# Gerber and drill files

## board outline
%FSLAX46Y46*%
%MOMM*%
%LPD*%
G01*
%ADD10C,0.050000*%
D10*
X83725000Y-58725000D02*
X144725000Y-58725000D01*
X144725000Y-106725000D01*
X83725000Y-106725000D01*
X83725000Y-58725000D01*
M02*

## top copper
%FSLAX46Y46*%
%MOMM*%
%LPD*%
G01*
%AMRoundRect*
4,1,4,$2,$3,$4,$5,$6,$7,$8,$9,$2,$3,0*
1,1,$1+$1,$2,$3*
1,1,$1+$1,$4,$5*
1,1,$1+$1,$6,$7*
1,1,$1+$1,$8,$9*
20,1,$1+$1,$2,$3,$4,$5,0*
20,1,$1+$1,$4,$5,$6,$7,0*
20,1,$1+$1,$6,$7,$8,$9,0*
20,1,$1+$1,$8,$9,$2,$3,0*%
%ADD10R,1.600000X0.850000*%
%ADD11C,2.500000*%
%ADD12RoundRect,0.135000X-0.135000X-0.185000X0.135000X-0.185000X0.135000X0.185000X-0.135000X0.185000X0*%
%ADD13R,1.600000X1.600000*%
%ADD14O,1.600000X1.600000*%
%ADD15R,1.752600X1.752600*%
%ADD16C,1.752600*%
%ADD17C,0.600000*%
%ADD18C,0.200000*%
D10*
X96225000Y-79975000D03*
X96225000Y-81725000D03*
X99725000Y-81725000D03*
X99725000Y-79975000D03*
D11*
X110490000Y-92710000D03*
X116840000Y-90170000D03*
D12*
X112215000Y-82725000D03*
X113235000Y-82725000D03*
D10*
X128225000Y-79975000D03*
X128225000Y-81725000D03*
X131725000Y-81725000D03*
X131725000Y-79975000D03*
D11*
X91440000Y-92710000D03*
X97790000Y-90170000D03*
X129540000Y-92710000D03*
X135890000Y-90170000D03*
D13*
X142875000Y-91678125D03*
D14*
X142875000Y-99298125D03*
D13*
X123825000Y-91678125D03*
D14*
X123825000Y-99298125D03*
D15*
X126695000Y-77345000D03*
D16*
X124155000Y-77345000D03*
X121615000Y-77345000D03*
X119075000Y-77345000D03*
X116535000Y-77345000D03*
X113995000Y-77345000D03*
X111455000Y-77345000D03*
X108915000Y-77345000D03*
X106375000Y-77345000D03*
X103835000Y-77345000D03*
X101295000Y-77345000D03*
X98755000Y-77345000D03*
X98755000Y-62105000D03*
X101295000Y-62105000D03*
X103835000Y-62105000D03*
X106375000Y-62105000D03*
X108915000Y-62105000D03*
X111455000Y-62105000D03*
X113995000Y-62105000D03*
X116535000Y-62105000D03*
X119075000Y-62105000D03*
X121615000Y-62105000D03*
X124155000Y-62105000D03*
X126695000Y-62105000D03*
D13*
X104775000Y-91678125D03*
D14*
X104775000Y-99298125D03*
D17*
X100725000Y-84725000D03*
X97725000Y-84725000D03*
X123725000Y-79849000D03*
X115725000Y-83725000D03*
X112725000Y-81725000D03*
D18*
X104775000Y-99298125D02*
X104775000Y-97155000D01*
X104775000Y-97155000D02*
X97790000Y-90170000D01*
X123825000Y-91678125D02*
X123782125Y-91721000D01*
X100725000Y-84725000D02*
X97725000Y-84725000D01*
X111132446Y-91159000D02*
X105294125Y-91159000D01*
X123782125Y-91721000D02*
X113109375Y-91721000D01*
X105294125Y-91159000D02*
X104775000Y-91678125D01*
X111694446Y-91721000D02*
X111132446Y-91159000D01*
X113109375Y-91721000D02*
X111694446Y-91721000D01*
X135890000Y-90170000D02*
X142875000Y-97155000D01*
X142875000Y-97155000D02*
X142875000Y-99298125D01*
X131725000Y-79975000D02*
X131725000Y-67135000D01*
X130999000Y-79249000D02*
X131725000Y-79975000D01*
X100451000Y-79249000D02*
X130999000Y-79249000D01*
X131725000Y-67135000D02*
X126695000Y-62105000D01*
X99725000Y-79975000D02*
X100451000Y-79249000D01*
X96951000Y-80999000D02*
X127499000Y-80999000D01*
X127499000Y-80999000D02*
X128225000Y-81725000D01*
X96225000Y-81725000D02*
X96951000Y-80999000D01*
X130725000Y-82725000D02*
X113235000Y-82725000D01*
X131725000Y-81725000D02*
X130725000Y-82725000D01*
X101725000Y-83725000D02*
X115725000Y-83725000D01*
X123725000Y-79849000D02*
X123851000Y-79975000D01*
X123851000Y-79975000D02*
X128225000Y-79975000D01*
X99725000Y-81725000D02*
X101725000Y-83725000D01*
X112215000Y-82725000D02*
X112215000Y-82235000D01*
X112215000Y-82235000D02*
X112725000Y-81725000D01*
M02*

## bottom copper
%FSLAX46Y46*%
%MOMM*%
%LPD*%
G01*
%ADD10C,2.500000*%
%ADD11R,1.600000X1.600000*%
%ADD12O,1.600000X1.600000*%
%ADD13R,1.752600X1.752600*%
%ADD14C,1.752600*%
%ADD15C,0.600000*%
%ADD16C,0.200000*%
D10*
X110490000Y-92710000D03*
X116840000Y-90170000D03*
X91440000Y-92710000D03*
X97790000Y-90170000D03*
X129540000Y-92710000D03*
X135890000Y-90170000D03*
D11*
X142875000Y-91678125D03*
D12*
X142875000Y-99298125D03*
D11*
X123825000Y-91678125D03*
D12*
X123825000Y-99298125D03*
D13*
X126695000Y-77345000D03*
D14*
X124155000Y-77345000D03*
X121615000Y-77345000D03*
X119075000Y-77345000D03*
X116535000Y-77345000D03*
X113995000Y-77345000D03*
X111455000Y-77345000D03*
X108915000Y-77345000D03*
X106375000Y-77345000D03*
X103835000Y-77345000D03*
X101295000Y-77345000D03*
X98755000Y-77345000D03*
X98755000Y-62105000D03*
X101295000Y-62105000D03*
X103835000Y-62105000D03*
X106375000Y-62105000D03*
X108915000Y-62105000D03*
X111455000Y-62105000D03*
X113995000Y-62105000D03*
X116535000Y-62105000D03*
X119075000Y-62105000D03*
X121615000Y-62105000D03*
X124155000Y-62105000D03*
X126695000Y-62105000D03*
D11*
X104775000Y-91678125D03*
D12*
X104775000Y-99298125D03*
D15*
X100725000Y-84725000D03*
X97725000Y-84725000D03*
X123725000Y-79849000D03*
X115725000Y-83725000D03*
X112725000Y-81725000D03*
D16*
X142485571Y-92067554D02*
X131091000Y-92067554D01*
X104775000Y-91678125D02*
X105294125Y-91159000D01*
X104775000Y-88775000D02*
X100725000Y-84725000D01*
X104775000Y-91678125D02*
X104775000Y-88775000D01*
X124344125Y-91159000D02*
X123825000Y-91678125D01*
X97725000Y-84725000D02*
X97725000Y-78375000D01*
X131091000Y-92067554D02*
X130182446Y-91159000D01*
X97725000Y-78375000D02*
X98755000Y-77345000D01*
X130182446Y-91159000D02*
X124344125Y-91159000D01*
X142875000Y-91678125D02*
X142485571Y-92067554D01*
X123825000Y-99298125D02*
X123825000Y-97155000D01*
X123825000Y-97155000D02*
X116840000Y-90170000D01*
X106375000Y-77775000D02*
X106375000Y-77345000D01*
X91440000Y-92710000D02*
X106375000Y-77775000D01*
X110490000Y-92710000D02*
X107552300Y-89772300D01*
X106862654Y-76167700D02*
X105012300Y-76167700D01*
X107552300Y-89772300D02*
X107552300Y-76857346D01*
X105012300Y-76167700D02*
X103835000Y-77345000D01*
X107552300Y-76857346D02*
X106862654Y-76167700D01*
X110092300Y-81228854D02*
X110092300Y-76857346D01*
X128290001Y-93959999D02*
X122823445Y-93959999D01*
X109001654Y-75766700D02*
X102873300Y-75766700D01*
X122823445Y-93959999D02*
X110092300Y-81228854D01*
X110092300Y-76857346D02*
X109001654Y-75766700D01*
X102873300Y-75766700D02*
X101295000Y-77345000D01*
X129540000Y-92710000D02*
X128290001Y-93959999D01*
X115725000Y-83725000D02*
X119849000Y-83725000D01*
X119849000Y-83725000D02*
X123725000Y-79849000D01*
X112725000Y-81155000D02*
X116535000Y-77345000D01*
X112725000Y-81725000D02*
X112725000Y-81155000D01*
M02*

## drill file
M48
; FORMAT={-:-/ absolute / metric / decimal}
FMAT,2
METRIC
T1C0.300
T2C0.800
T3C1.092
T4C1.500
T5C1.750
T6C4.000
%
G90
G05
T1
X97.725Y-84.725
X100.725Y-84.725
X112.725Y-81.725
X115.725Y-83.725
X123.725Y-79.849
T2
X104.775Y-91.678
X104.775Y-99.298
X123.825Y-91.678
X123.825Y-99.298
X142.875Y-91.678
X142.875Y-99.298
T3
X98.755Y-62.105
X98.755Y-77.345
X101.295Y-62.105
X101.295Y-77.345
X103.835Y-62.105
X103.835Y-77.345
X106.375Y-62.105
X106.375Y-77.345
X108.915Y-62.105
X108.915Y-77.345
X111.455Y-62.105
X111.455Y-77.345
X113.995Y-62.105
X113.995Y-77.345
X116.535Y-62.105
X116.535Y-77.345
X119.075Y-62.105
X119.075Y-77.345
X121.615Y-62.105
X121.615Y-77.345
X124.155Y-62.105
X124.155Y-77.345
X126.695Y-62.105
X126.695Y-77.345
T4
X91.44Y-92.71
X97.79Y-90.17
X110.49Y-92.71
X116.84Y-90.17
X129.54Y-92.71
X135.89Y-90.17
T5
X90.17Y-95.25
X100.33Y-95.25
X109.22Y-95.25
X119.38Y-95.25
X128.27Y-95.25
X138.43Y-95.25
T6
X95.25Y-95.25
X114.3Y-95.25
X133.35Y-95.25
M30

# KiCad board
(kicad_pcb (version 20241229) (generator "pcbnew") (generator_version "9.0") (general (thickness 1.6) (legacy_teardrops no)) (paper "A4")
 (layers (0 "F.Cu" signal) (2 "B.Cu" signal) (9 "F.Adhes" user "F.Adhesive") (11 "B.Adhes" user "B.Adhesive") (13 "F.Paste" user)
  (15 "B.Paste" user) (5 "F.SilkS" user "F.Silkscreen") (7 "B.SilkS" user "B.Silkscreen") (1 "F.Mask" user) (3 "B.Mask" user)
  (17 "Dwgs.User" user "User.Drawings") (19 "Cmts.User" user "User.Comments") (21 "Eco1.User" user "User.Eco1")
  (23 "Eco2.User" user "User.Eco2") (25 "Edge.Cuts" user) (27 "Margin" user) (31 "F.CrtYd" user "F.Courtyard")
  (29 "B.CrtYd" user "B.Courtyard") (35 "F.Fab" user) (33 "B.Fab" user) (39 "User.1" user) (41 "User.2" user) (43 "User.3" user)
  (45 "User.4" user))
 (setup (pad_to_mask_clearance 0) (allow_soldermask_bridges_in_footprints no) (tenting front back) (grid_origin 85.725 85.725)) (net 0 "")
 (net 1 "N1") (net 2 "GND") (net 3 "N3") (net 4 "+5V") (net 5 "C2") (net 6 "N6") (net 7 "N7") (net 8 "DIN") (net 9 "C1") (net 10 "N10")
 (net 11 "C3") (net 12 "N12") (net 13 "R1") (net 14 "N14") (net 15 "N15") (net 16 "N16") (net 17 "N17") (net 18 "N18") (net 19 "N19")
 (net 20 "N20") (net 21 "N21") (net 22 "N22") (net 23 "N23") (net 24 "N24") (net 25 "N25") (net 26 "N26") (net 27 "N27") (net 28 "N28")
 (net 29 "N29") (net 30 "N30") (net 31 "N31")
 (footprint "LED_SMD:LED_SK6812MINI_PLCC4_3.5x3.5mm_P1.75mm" (layer "F.Cu") (at 97.975 80.85)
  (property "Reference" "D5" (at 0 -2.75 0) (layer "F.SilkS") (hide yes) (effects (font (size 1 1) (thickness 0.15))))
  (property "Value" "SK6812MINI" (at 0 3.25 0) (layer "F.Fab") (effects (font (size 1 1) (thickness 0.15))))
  (pad "1" smd rect (at -1.75 -0.875) (size 1.6 0.85) (layers "F.Cu" "F.Mask" "F.Paste") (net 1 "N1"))
  (pad "2" smd rect (at -1.75 0.875) (size 1.6 0.85) (layers "F.Cu" "F.Mask" "F.Paste") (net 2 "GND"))
  (pad "3" smd rect (at 1.75 0.875) (size 1.6 0.85) (layers "F.Cu" "F.Mask" "F.Paste") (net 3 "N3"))
  (pad "4" smd rect (at 1.75 -0.875) (size 1.6 0.85) (layers "F.Cu" "F.Mask" "F.Paste") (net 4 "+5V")))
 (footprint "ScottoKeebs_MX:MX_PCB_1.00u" (layer "F.Cu") (at 114.3 95.25)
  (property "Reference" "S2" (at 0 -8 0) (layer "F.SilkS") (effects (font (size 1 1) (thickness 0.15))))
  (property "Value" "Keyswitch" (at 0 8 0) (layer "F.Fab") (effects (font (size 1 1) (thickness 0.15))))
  (pad "" np_thru_hole circle (at -5.08 0) (size 1.75 1.75) (drill 1.75) (layers "*.Cu" "*.Mask"))
  (pad "" np_thru_hole circle (at 0 0) (size 4 4) (drill 4) (layers "*.Cu" "*.Mask"))
  (pad "" np_thru_hole circle (at 5.08 0) (size 1.75 1.75) (drill 1.75) (layers "*.Cu" "*.Mask"))
  (pad "1" thru_hole circle (at -3.81 -2.54) (size 2.5 2.5) (drill 1.5) (layers "*.Cu" "*.Mask") (remove_unused_layers no) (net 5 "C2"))
  (pad "2" thru_hole circle (at 2.54 -5.08) (size 2.5 2.5) (drill 1.5) (layers "*.Cu" "*.Mask") (remove_unused_layers no) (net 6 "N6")))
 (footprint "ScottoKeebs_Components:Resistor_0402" (layer "F.Cu") (at 112.725 82.725)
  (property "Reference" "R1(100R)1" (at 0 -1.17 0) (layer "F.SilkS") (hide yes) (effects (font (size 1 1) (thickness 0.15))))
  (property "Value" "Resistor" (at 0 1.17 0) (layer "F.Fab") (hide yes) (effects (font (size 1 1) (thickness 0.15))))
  (pad "1" smd roundrect (at -0.51 0) (size 0.54 0.64) (layers "F.Cu" "F.Mask" "F.Paste") (roundrect_rratio 0.25) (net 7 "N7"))
  (pad "2" smd roundrect (at 0.51 0) (size 0.54 0.64) (layers "F.Cu" "F.Mask" "F.Paste") (roundrect_rratio 0.25) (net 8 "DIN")))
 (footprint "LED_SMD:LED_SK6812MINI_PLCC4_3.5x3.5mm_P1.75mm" (layer "F.Cu") (at 129.975 80.85)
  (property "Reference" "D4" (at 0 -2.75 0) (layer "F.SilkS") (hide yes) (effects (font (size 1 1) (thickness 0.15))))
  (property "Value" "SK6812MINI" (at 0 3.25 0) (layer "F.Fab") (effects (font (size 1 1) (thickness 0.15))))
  (pad "1" smd rect (at -1.75 -0.875) (size 1.6 0.85) (layers "F.Cu" "F.Mask" "F.Paste") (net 3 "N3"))
  (pad "2" smd rect (at -1.75 0.875) (size 1.6 0.85) (layers "F.Cu" "F.Mask" "F.Paste") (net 2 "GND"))
  (pad "3" smd rect (at 1.75 0.875) (size 1.6 0.85) (layers "F.Cu" "F.Mask" "F.Paste") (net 8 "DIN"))
  (pad "4" smd rect (at 1.75 -0.875) (size 1.6 0.85) (layers "F.Cu" "F.Mask" "F.Paste") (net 4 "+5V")))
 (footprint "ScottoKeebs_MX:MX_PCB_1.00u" (layer "F.Cu") (at 95.25 95.25)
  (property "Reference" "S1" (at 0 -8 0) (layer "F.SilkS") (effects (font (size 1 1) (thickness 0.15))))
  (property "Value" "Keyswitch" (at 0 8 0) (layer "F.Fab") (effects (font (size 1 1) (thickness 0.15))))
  (pad "" np_thru_hole circle (at -5.08 0) (size 1.75 1.75) (drill 1.75) (layers "*.Cu" "*.Mask"))
  (pad "" np_thru_hole circle (at 0 0) (size 4 4) (drill 4) (layers "*.Cu" "*.Mask"))
  (pad "" np_thru_hole circle (at 5.08 0) (size 1.75 1.75) (drill 1.75) (layers "*.Cu" "*.Mask"))
  (pad "1" thru_hole circle (at -3.81 -2.54) (size 2.5 2.5) (drill 1.5) (layers "*.Cu" "*.Mask") (remove_unused_layers no) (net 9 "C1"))
  (pad "2" thru_hole circle (at 2.54 -5.08) (size 2.5 2.5) (drill 1.5) (layers "*.Cu" "*.Mask") (remove_unused_layers no) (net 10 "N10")))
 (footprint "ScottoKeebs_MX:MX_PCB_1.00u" (layer "F.Cu") (at 133.35 95.25)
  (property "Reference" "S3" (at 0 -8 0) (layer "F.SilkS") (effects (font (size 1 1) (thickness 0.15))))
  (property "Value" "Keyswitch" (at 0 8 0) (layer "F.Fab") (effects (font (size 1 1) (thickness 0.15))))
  (pad "" np_thru_hole circle (at -5.08 0) (size 1.75 1.75) (drill 1.75) (layers "*.Cu" "*.Mask"))
  (pad "" np_thru_hole circle (at 0 0) (size 4 4) (drill 4) (layers "*.Cu" "*.Mask"))
  (pad "" np_thru_hole circle (at 5.08 0) (size 1.75 1.75) (drill 1.75) (layers "*.Cu" "*.Mask"))
  (pad "1" thru_hole circle (at -3.81 -2.54) (size 2.5 2.5) (drill 1.5) (layers "*.Cu" "*.Mask") (remove_unused_layers no) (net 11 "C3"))
  (pad "2" thru_hole circle (at 2.54 -5.08) (size 2.5 2.5) (drill 1.5) (layers "*.Cu" "*.Mask") (remove_unused_layers no) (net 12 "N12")))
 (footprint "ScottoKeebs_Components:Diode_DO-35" (layer "B.Cu") (at 142.875 91.678125 -90)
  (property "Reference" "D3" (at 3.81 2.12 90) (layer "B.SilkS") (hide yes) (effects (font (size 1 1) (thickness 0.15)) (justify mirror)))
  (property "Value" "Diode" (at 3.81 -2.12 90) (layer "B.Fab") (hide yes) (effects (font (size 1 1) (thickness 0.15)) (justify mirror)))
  (pad "1" thru_hole rect (at 0 0 270) (size 1.6 1.6) (drill 0.8) (layers "*.Cu" "*.Mask") (remove_unused_layers no) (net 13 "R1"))
  (pad "2" thru_hole oval (at 7.62 0 270) (size 1.6 1.6) (drill 0.8) (layers "*.Cu" "*.Mask") (remove_unused_layers no) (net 12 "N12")))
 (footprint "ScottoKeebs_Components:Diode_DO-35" (layer "B.Cu") (at 123.825 91.678125 -90)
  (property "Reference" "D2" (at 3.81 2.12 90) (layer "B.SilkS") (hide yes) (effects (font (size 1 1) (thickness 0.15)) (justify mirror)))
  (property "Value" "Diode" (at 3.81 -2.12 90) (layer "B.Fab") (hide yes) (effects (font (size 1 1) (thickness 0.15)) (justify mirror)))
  (pad "1" thru_hole rect (at 0 0 270) (size 1.6 1.6) (drill 0.8) (layers "*.Cu" "*.Mask") (remove_unused_layers no) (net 13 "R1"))
  (pad "2" thru_hole oval (at 7.62 0 270) (size 1.6 1.6) (drill 0.8) (layers "*.Cu" "*.Mask") (remove_unused_layers no) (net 6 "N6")))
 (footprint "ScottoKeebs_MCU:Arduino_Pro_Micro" (layer "B.Cu") (at 112.725 69.725 90)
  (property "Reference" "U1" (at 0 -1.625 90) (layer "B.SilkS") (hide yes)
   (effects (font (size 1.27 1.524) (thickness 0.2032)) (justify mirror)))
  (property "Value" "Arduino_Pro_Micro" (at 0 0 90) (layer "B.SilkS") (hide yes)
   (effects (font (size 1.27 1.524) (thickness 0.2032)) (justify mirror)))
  (pad "1" thru_hole rect (at -7.62 13.97 180) (size 1.7526 1.7526) (drill 1.0922) (layers "*.Cu" "*.SilkS" "*.Mask")
   (remove_unused_layers no) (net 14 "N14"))
  (pad "2" thru_hole circle (at -7.62 11.43 180) (size 1.7526 1.7526) (drill 1.0922) (layers "*.Cu" "*.SilkS" "*.Mask")
   (remove_unused_layers no) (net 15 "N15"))
  (pad "3" thru_hole circle (at -7.62 8.89 180) (size 1.7526 1.7526) (drill 1.0922) (layers "*.Cu" "*.SilkS" "*.Mask")
   (remove_unused_layers no) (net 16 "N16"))
  (pad "4" thru_hole circle (at -7.62 6.35 180) (size 1.7526 1.7526) (drill 1.0922) (layers "*.Cu" "*.SilkS" "*.Mask")
   (remove_unused_layers no) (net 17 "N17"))
  (pad "5" thru_hole circle (at -7.62 3.81 180) (size 1.7526 1.7526) (drill 1.0922) (layers "*.Cu" "*.SilkS" "*.Mask")
   (remove_unused_layers no) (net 7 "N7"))
  (pad "6" thru_hole circle (at -7.62 1.27 180) (size 1.7526 1.7526) (drill 1.0922) (layers "*.Cu" "*.SilkS" "*.Mask")
   (remove_unused_layers no) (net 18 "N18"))
  (pad "7" thru_hole circle (at -7.62 -1.27 180) (size 1.7526 1.7526) (drill 1.0922) (layers "*.Cu" "*.SilkS" "*.Mask")
   (remove_unused_layers no) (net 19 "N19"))
  (pad "8" thru_hole circle (at -7.62 -3.81 180) (size 1.7526 1.7526) (drill 1.0922) (layers "*.Cu" "*.SilkS" "*.Mask")
   (remove_unused_layers no) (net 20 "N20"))
  (pad "9" thru_hole circle (at -7.62 -6.35 180) (size 1.7526 1.7526) (drill 1.0922) (layers "*.Cu" "*.SilkS" "*.Mask")
   (remove_unused_layers no) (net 9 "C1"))
  (pad "10" thru_hole circle (at -7.62 -8.89 180) (size 1.7526 1.7526) (drill 1.0922) (layers "*.Cu" "*.SilkS" "*.Mask")
   (remove_unused_layers no) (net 5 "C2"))
  (pad "11" thru_hole circle (at -7.62 -11.43 180) (size 1.7526 1.7526) (drill 1.0922) (layers "*.Cu" "*.SilkS" "*.Mask")
   (remove_unused_layers no) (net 11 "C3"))
  (pad "12" thru_hole circle (at -7.62 -13.97 180) (size 1.7526 1.7526) (drill 1.0922) (layers "*.Cu" "*.SilkS" "*.Mask")
   (remove_unused_layers no) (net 13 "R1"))
  (pad "13" thru_hole circle (at 7.62 -13.97 180) (size 1.7526 1.7526) (drill 1.0922) (layers "*.Cu" "*.SilkS" "*.Mask")
   (remove_unused_layers no) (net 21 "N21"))
  (pad "14" thru_hole circle (at 7.62 -11.43 180) (size 1.7526 1.7526) (drill 1.0922) (layers "*.Cu" "*.SilkS" "*.Mask")
   (remove_unused_layers no) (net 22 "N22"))
  (pad "15" thru_hole circle (at 7.62 -8.89 180) (size 1.7526 1.7526) (drill 1.0922) (layers "*.Cu" "*.SilkS" "*.Mask")
   (remove_unused_layers no) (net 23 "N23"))
  (pad "16" thru_hole circle (at 7.62 -6.35 180) (size 1.7526 1.7526) (drill 1.0922) (layers "*.Cu" "*.SilkS" "*.Mask")
   (remove_unused_layers no) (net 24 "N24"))
  (pad "17" thru_hole circle (at 7.62 -3.81 180) (size 1.7526 1.7526) (drill 1.0922) (layers "*.Cu" "*.SilkS" "*.Mask")
   (remove_unused_layers no) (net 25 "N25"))
  (pad "18" thru_hole circle (at 7.62 -1.27 180) (size 1.7526 1.7526) (drill 1.0922) (layers "*.Cu" "*.SilkS" "*.Mask")
   (remove_unused_layers no) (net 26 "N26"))
  (pad "19" thru_hole circle (at 7.62 1.27 180) (size 1.7526 1.7526) (drill 1.0922) (layers "*.Cu" "*.SilkS" "*.Mask")
   (remove_unused_layers no) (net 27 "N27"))
  (pad "20" thru_hole circle (at 7.62 3.81 180) (size 1.7526 1.7526) (drill 1.0922) (layers "*.Cu" "*.SilkS" "*.Mask")
   (remove_unused_layers no) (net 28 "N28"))
  (pad "21" thru_hole circle (at 7.62 6.35 180) (size 1.7526 1.7526) (drill 1.0922) (layers "*.Cu" "*.SilkS" "*.Mask")
   (remove_unused_layers no) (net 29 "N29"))
  (pad "22" thru_hole circle (at 7.62 8.89 180) (size 1.7526 1.7526) (drill 1.0922) (layers "*.Cu" "*.SilkS" "*.Mask")
   (remove_unused_layers no) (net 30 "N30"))
  (pad "23" thru_hole circle (at 7.62 11.43 180) (size 1.7526 1.7526) (drill 1.0922) (layers "*.Cu" "*.SilkS" "*.Mask")
   (remove_unused_layers no) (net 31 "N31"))
  (pad "24" thru_hole circle (at 7.62 13.97 180) (size 1.7526 1.7526) (drill 1.0922) (layers "*.Cu" "*.SilkS" "*.Mask")
   (remove_unused_layers no) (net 4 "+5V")))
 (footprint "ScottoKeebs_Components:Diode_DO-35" (layer "B.Cu") (at 104.775 91.678125 -90)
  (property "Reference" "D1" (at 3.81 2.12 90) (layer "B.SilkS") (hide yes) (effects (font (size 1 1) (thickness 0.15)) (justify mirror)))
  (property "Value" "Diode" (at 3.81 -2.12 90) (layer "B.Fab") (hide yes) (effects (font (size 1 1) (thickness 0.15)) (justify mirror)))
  (pad "1" thru_hole rect (at 0 0 270) (size 1.6 1.6) (drill 0.8) (layers "*.Cu" "*.Mask") (remove_unused_layers no) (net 13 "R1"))
  (pad "2" thru_hole oval (at 7.62 0 270) (size 1.6 1.6) (drill 0.8) (layers "*.Cu" "*.Mask") (remove_unused_layers no) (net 10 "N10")))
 (gr_rect (start 83.725 58.725) (end 144.725 106.725) (stroke (width 0.05) (type default)) (fill no) (layer "Edge.Cuts"))
 (segment (start 104.775 99.298125) (end 104.775 97.155) (width 0.2) (layer "F.Cu") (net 10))
 (segment (start 104.775 97.155) (end 97.79 90.17) (width 0.2) (layer "F.Cu") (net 10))
 (segment (start 123.825 91.678125) (end 123.782125 91.721) (width 0.2) (layer "F.Cu") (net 13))
 (segment (start 100.725 84.725) (end 97.725 84.725) (width 0.2) (layer "F.Cu") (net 13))
 (segment (start 111.132446 91.159) (end 105.294125 91.159) (width 0.2) (layer "F.Cu") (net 13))
 (segment (start 123.782125 91.721) (end 113.109375 91.721) (width 0.2) (layer "F.Cu") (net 13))
 (segment (start 105.294125 91.159) (end 104.775 91.678125) (width 0.2) (layer "F.Cu") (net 13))
 (segment (start 111.694446 91.721) (end 111.132446 91.159) (width 0.2) (layer "F.Cu") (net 13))
 (segment (start 113.109375 91.721) (end 111.694446 91.721) (width 0.2) (layer "F.Cu") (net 13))
 (via (at 100.725 84.725) (size 0.6) (drill 0.3) (layers "F.Cu" "B.Cu") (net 13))
 (via (at 97.725 84.725) (size 0.6) (drill 0.3) (layers "F.Cu" "B.Cu") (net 13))
 (segment (start 142.485571 92.067554) (end 131.091 92.067554) (width 0.2) (layer "B.Cu") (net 13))
 (segment (start 104.775 91.678125) (end 105.294125 91.159) (width 0.2) (layer "B.Cu") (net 13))
 (segment (start 104.775 88.775) (end 100.725 84.725) (width 0.2) (layer "B.Cu") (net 13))
 (segment (start 104.775 91.678125) (end 104.775 88.775) (width 0.2) (layer "B.Cu") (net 13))
 (segment (start 124.344125 91.159) (end 123.825 91.678125) (width 0.2) (layer "B.Cu") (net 13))
 (segment (start 97.725 84.725) (end 97.725 78.375) (width 0.2) (layer "B.Cu") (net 13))
 (segment (start 131.091 92.067554) (end 130.182446 91.159) (width 0.2) (layer "B.Cu") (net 13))
 (segment (start 97.725 78.375) (end 98.755 77.345) (width 0.2) (layer "B.Cu") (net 13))
 (segment (start 130.182446 91.159) (end 124.344125 91.159) (width 0.2) (layer "B.Cu") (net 13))
 (segment (start 142.875 91.678125) (end 142.485571 92.067554) (width 0.2) (layer "B.Cu") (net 13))
 (segment (start 123.825 99.298125) (end 123.825 97.155) (width 0.2) (layer "B.Cu") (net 6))
 (segment (start 123.825 97.155) (end 116.84 90.17) (width 0.2) (layer "B.Cu") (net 6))
 (segment (start 135.89 90.17) (end 142.875 97.155) (width 0.2) (layer "F.Cu") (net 12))
 (segment (start 142.875 97.155) (end 142.875 99.298125) (width 0.2) (layer "F.Cu") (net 12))
 (segment (start 106.375 77.775) (end 106.375 77.345) (width 0.2) (layer "B.Cu") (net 9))
 (segment (start 91.44 92.71) (end 106.375 77.775) (width 0.2) (layer "B.Cu") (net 9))
 (segment (start 110.49 92.71) (end 107.5523 89.7723) (width 0.2) (layer "B.Cu") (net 5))
 (segment (start 106.862654 76.1677) (end 105.0123 76.1677) (width 0.2) (layer "B.Cu") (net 5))
 (segment (start 107.5523 89.7723) (end 107.5523 76.857346) (width 0.2) (layer "B.Cu") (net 5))
 (segment (start 105.0123 76.1677) (end 103.835 77.345) (width 0.2) (layer "B.Cu") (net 5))
 (segment (start 107.5523 76.857346) (end 106.862654 76.1677) (width 0.2) (layer "B.Cu") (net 5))
 (segment (start 110.0923 81.228854) (end 110.0923 76.857346) (width 0.2) (layer "B.Cu") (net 11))
 (segment (start 128.290001 93.959999) (end 122.823445 93.959999) (width 0.2) (layer "B.Cu") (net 11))
 (segment (start 109.001654 75.7667) (end 102.8733 75.7667) (width 0.2) (layer "B.Cu") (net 11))
 (segment (start 122.823445 93.959999) (end 110.0923 81.228854) (width 0.2) (layer "B.Cu") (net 11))
 (segment (start 110.0923 76.857346) (end 109.001654 75.7667) (width 0.2) (layer "B.Cu") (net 11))
 (segment (start 102.8733 75.7667) (end 101.295 77.345) (width 0.2) (layer "B.Cu") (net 11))
 (segment (start 129.54 92.71) (end 128.290001 93.959999) (width 0.2) (layer "B.Cu") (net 11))
 (segment (start 131.725 79.975) (end 131.725 67.135) (width 0.2) (layer "F.Cu") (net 4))
 (segment (start 130.999 79.249) (end 131.725 79.975) (width 0.2) (layer "F.Cu") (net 4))
 (segment (start 100.451 79.249) (end 130.999 79.249) (width 0.2) (layer "F.Cu") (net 4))
 (segment (start 131.725 67.135) (end 126.695 62.105) (width 0.2) (layer "F.Cu") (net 4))
 (segment (start 99.725 79.975) (end 100.451 79.249) (width 0.2) (layer "F.Cu") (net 4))
 (segment (start 96.951 80.999) (end 127.499 80.999) (width 0.2) (layer "F.Cu") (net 2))
 (segment (start 127.499 80.999) (end 128.225 81.725) (width 0.2) (layer "F.Cu") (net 2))
 (segment (start 96.225 81.725) (end 96.951 80.999) (width 0.2) (layer "F.Cu") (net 2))
 (segment (start 130.725 82.725) (end 113.235 82.725) (width 0.2) (layer "F.Cu") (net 8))
 (segment (start 131.725 81.725) (end 130.725 82.725) (width 0.2) (layer "F.Cu") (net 8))
 (segment (start 101.725 83.725) (end 115.725 83.725) (width 0.2) (layer "F.Cu") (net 3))
 (segment (start 123.725 79.849) (end 123.851 79.975) (width 0.2) (layer "F.Cu") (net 3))
 (segment (start 123.851 79.975) (end 128.225 79.975) (width 0.2) (layer "F.Cu") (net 3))
 (segment (start 99.725 81.725) (end 101.725 83.725) (width 0.2) (layer "F.Cu") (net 3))
 (via (at 123.725 79.849) (size 0.6) (drill 0.3) (layers "F.Cu" "B.Cu") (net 3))
 (via (at 115.725 83.725) (size 0.6) (drill 0.3) (layers "F.Cu" "B.Cu") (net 3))
 (segment (start 115.725 83.725) (end 119.849 83.725) (width 0.2) (layer "B.Cu") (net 3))
 (segment (start 119.849 83.725) (end 123.725 79.849) (width 0.2) (layer "B.Cu") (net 3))
 (segment (start 112.215 82.725) (end 112.215 82.235) (width 0.2) (layer "F.Cu") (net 7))
 (segment (start 112.215 82.235) (end 112.725 81.725) (width 0.2) (layer "F.Cu") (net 7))
 (via (at 112.725 81.725) (size 0.6) (drill 0.3) (layers "F.Cu" "B.Cu") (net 7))
 (segment (start 112.725 81.155) (end 116.535 77.345) (width 0.2) (layer "B.Cu") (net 7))
 (segment (start 112.725 81.725) (end 112.725 81.155) (width 0.2) (layer "B.Cu") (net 7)))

